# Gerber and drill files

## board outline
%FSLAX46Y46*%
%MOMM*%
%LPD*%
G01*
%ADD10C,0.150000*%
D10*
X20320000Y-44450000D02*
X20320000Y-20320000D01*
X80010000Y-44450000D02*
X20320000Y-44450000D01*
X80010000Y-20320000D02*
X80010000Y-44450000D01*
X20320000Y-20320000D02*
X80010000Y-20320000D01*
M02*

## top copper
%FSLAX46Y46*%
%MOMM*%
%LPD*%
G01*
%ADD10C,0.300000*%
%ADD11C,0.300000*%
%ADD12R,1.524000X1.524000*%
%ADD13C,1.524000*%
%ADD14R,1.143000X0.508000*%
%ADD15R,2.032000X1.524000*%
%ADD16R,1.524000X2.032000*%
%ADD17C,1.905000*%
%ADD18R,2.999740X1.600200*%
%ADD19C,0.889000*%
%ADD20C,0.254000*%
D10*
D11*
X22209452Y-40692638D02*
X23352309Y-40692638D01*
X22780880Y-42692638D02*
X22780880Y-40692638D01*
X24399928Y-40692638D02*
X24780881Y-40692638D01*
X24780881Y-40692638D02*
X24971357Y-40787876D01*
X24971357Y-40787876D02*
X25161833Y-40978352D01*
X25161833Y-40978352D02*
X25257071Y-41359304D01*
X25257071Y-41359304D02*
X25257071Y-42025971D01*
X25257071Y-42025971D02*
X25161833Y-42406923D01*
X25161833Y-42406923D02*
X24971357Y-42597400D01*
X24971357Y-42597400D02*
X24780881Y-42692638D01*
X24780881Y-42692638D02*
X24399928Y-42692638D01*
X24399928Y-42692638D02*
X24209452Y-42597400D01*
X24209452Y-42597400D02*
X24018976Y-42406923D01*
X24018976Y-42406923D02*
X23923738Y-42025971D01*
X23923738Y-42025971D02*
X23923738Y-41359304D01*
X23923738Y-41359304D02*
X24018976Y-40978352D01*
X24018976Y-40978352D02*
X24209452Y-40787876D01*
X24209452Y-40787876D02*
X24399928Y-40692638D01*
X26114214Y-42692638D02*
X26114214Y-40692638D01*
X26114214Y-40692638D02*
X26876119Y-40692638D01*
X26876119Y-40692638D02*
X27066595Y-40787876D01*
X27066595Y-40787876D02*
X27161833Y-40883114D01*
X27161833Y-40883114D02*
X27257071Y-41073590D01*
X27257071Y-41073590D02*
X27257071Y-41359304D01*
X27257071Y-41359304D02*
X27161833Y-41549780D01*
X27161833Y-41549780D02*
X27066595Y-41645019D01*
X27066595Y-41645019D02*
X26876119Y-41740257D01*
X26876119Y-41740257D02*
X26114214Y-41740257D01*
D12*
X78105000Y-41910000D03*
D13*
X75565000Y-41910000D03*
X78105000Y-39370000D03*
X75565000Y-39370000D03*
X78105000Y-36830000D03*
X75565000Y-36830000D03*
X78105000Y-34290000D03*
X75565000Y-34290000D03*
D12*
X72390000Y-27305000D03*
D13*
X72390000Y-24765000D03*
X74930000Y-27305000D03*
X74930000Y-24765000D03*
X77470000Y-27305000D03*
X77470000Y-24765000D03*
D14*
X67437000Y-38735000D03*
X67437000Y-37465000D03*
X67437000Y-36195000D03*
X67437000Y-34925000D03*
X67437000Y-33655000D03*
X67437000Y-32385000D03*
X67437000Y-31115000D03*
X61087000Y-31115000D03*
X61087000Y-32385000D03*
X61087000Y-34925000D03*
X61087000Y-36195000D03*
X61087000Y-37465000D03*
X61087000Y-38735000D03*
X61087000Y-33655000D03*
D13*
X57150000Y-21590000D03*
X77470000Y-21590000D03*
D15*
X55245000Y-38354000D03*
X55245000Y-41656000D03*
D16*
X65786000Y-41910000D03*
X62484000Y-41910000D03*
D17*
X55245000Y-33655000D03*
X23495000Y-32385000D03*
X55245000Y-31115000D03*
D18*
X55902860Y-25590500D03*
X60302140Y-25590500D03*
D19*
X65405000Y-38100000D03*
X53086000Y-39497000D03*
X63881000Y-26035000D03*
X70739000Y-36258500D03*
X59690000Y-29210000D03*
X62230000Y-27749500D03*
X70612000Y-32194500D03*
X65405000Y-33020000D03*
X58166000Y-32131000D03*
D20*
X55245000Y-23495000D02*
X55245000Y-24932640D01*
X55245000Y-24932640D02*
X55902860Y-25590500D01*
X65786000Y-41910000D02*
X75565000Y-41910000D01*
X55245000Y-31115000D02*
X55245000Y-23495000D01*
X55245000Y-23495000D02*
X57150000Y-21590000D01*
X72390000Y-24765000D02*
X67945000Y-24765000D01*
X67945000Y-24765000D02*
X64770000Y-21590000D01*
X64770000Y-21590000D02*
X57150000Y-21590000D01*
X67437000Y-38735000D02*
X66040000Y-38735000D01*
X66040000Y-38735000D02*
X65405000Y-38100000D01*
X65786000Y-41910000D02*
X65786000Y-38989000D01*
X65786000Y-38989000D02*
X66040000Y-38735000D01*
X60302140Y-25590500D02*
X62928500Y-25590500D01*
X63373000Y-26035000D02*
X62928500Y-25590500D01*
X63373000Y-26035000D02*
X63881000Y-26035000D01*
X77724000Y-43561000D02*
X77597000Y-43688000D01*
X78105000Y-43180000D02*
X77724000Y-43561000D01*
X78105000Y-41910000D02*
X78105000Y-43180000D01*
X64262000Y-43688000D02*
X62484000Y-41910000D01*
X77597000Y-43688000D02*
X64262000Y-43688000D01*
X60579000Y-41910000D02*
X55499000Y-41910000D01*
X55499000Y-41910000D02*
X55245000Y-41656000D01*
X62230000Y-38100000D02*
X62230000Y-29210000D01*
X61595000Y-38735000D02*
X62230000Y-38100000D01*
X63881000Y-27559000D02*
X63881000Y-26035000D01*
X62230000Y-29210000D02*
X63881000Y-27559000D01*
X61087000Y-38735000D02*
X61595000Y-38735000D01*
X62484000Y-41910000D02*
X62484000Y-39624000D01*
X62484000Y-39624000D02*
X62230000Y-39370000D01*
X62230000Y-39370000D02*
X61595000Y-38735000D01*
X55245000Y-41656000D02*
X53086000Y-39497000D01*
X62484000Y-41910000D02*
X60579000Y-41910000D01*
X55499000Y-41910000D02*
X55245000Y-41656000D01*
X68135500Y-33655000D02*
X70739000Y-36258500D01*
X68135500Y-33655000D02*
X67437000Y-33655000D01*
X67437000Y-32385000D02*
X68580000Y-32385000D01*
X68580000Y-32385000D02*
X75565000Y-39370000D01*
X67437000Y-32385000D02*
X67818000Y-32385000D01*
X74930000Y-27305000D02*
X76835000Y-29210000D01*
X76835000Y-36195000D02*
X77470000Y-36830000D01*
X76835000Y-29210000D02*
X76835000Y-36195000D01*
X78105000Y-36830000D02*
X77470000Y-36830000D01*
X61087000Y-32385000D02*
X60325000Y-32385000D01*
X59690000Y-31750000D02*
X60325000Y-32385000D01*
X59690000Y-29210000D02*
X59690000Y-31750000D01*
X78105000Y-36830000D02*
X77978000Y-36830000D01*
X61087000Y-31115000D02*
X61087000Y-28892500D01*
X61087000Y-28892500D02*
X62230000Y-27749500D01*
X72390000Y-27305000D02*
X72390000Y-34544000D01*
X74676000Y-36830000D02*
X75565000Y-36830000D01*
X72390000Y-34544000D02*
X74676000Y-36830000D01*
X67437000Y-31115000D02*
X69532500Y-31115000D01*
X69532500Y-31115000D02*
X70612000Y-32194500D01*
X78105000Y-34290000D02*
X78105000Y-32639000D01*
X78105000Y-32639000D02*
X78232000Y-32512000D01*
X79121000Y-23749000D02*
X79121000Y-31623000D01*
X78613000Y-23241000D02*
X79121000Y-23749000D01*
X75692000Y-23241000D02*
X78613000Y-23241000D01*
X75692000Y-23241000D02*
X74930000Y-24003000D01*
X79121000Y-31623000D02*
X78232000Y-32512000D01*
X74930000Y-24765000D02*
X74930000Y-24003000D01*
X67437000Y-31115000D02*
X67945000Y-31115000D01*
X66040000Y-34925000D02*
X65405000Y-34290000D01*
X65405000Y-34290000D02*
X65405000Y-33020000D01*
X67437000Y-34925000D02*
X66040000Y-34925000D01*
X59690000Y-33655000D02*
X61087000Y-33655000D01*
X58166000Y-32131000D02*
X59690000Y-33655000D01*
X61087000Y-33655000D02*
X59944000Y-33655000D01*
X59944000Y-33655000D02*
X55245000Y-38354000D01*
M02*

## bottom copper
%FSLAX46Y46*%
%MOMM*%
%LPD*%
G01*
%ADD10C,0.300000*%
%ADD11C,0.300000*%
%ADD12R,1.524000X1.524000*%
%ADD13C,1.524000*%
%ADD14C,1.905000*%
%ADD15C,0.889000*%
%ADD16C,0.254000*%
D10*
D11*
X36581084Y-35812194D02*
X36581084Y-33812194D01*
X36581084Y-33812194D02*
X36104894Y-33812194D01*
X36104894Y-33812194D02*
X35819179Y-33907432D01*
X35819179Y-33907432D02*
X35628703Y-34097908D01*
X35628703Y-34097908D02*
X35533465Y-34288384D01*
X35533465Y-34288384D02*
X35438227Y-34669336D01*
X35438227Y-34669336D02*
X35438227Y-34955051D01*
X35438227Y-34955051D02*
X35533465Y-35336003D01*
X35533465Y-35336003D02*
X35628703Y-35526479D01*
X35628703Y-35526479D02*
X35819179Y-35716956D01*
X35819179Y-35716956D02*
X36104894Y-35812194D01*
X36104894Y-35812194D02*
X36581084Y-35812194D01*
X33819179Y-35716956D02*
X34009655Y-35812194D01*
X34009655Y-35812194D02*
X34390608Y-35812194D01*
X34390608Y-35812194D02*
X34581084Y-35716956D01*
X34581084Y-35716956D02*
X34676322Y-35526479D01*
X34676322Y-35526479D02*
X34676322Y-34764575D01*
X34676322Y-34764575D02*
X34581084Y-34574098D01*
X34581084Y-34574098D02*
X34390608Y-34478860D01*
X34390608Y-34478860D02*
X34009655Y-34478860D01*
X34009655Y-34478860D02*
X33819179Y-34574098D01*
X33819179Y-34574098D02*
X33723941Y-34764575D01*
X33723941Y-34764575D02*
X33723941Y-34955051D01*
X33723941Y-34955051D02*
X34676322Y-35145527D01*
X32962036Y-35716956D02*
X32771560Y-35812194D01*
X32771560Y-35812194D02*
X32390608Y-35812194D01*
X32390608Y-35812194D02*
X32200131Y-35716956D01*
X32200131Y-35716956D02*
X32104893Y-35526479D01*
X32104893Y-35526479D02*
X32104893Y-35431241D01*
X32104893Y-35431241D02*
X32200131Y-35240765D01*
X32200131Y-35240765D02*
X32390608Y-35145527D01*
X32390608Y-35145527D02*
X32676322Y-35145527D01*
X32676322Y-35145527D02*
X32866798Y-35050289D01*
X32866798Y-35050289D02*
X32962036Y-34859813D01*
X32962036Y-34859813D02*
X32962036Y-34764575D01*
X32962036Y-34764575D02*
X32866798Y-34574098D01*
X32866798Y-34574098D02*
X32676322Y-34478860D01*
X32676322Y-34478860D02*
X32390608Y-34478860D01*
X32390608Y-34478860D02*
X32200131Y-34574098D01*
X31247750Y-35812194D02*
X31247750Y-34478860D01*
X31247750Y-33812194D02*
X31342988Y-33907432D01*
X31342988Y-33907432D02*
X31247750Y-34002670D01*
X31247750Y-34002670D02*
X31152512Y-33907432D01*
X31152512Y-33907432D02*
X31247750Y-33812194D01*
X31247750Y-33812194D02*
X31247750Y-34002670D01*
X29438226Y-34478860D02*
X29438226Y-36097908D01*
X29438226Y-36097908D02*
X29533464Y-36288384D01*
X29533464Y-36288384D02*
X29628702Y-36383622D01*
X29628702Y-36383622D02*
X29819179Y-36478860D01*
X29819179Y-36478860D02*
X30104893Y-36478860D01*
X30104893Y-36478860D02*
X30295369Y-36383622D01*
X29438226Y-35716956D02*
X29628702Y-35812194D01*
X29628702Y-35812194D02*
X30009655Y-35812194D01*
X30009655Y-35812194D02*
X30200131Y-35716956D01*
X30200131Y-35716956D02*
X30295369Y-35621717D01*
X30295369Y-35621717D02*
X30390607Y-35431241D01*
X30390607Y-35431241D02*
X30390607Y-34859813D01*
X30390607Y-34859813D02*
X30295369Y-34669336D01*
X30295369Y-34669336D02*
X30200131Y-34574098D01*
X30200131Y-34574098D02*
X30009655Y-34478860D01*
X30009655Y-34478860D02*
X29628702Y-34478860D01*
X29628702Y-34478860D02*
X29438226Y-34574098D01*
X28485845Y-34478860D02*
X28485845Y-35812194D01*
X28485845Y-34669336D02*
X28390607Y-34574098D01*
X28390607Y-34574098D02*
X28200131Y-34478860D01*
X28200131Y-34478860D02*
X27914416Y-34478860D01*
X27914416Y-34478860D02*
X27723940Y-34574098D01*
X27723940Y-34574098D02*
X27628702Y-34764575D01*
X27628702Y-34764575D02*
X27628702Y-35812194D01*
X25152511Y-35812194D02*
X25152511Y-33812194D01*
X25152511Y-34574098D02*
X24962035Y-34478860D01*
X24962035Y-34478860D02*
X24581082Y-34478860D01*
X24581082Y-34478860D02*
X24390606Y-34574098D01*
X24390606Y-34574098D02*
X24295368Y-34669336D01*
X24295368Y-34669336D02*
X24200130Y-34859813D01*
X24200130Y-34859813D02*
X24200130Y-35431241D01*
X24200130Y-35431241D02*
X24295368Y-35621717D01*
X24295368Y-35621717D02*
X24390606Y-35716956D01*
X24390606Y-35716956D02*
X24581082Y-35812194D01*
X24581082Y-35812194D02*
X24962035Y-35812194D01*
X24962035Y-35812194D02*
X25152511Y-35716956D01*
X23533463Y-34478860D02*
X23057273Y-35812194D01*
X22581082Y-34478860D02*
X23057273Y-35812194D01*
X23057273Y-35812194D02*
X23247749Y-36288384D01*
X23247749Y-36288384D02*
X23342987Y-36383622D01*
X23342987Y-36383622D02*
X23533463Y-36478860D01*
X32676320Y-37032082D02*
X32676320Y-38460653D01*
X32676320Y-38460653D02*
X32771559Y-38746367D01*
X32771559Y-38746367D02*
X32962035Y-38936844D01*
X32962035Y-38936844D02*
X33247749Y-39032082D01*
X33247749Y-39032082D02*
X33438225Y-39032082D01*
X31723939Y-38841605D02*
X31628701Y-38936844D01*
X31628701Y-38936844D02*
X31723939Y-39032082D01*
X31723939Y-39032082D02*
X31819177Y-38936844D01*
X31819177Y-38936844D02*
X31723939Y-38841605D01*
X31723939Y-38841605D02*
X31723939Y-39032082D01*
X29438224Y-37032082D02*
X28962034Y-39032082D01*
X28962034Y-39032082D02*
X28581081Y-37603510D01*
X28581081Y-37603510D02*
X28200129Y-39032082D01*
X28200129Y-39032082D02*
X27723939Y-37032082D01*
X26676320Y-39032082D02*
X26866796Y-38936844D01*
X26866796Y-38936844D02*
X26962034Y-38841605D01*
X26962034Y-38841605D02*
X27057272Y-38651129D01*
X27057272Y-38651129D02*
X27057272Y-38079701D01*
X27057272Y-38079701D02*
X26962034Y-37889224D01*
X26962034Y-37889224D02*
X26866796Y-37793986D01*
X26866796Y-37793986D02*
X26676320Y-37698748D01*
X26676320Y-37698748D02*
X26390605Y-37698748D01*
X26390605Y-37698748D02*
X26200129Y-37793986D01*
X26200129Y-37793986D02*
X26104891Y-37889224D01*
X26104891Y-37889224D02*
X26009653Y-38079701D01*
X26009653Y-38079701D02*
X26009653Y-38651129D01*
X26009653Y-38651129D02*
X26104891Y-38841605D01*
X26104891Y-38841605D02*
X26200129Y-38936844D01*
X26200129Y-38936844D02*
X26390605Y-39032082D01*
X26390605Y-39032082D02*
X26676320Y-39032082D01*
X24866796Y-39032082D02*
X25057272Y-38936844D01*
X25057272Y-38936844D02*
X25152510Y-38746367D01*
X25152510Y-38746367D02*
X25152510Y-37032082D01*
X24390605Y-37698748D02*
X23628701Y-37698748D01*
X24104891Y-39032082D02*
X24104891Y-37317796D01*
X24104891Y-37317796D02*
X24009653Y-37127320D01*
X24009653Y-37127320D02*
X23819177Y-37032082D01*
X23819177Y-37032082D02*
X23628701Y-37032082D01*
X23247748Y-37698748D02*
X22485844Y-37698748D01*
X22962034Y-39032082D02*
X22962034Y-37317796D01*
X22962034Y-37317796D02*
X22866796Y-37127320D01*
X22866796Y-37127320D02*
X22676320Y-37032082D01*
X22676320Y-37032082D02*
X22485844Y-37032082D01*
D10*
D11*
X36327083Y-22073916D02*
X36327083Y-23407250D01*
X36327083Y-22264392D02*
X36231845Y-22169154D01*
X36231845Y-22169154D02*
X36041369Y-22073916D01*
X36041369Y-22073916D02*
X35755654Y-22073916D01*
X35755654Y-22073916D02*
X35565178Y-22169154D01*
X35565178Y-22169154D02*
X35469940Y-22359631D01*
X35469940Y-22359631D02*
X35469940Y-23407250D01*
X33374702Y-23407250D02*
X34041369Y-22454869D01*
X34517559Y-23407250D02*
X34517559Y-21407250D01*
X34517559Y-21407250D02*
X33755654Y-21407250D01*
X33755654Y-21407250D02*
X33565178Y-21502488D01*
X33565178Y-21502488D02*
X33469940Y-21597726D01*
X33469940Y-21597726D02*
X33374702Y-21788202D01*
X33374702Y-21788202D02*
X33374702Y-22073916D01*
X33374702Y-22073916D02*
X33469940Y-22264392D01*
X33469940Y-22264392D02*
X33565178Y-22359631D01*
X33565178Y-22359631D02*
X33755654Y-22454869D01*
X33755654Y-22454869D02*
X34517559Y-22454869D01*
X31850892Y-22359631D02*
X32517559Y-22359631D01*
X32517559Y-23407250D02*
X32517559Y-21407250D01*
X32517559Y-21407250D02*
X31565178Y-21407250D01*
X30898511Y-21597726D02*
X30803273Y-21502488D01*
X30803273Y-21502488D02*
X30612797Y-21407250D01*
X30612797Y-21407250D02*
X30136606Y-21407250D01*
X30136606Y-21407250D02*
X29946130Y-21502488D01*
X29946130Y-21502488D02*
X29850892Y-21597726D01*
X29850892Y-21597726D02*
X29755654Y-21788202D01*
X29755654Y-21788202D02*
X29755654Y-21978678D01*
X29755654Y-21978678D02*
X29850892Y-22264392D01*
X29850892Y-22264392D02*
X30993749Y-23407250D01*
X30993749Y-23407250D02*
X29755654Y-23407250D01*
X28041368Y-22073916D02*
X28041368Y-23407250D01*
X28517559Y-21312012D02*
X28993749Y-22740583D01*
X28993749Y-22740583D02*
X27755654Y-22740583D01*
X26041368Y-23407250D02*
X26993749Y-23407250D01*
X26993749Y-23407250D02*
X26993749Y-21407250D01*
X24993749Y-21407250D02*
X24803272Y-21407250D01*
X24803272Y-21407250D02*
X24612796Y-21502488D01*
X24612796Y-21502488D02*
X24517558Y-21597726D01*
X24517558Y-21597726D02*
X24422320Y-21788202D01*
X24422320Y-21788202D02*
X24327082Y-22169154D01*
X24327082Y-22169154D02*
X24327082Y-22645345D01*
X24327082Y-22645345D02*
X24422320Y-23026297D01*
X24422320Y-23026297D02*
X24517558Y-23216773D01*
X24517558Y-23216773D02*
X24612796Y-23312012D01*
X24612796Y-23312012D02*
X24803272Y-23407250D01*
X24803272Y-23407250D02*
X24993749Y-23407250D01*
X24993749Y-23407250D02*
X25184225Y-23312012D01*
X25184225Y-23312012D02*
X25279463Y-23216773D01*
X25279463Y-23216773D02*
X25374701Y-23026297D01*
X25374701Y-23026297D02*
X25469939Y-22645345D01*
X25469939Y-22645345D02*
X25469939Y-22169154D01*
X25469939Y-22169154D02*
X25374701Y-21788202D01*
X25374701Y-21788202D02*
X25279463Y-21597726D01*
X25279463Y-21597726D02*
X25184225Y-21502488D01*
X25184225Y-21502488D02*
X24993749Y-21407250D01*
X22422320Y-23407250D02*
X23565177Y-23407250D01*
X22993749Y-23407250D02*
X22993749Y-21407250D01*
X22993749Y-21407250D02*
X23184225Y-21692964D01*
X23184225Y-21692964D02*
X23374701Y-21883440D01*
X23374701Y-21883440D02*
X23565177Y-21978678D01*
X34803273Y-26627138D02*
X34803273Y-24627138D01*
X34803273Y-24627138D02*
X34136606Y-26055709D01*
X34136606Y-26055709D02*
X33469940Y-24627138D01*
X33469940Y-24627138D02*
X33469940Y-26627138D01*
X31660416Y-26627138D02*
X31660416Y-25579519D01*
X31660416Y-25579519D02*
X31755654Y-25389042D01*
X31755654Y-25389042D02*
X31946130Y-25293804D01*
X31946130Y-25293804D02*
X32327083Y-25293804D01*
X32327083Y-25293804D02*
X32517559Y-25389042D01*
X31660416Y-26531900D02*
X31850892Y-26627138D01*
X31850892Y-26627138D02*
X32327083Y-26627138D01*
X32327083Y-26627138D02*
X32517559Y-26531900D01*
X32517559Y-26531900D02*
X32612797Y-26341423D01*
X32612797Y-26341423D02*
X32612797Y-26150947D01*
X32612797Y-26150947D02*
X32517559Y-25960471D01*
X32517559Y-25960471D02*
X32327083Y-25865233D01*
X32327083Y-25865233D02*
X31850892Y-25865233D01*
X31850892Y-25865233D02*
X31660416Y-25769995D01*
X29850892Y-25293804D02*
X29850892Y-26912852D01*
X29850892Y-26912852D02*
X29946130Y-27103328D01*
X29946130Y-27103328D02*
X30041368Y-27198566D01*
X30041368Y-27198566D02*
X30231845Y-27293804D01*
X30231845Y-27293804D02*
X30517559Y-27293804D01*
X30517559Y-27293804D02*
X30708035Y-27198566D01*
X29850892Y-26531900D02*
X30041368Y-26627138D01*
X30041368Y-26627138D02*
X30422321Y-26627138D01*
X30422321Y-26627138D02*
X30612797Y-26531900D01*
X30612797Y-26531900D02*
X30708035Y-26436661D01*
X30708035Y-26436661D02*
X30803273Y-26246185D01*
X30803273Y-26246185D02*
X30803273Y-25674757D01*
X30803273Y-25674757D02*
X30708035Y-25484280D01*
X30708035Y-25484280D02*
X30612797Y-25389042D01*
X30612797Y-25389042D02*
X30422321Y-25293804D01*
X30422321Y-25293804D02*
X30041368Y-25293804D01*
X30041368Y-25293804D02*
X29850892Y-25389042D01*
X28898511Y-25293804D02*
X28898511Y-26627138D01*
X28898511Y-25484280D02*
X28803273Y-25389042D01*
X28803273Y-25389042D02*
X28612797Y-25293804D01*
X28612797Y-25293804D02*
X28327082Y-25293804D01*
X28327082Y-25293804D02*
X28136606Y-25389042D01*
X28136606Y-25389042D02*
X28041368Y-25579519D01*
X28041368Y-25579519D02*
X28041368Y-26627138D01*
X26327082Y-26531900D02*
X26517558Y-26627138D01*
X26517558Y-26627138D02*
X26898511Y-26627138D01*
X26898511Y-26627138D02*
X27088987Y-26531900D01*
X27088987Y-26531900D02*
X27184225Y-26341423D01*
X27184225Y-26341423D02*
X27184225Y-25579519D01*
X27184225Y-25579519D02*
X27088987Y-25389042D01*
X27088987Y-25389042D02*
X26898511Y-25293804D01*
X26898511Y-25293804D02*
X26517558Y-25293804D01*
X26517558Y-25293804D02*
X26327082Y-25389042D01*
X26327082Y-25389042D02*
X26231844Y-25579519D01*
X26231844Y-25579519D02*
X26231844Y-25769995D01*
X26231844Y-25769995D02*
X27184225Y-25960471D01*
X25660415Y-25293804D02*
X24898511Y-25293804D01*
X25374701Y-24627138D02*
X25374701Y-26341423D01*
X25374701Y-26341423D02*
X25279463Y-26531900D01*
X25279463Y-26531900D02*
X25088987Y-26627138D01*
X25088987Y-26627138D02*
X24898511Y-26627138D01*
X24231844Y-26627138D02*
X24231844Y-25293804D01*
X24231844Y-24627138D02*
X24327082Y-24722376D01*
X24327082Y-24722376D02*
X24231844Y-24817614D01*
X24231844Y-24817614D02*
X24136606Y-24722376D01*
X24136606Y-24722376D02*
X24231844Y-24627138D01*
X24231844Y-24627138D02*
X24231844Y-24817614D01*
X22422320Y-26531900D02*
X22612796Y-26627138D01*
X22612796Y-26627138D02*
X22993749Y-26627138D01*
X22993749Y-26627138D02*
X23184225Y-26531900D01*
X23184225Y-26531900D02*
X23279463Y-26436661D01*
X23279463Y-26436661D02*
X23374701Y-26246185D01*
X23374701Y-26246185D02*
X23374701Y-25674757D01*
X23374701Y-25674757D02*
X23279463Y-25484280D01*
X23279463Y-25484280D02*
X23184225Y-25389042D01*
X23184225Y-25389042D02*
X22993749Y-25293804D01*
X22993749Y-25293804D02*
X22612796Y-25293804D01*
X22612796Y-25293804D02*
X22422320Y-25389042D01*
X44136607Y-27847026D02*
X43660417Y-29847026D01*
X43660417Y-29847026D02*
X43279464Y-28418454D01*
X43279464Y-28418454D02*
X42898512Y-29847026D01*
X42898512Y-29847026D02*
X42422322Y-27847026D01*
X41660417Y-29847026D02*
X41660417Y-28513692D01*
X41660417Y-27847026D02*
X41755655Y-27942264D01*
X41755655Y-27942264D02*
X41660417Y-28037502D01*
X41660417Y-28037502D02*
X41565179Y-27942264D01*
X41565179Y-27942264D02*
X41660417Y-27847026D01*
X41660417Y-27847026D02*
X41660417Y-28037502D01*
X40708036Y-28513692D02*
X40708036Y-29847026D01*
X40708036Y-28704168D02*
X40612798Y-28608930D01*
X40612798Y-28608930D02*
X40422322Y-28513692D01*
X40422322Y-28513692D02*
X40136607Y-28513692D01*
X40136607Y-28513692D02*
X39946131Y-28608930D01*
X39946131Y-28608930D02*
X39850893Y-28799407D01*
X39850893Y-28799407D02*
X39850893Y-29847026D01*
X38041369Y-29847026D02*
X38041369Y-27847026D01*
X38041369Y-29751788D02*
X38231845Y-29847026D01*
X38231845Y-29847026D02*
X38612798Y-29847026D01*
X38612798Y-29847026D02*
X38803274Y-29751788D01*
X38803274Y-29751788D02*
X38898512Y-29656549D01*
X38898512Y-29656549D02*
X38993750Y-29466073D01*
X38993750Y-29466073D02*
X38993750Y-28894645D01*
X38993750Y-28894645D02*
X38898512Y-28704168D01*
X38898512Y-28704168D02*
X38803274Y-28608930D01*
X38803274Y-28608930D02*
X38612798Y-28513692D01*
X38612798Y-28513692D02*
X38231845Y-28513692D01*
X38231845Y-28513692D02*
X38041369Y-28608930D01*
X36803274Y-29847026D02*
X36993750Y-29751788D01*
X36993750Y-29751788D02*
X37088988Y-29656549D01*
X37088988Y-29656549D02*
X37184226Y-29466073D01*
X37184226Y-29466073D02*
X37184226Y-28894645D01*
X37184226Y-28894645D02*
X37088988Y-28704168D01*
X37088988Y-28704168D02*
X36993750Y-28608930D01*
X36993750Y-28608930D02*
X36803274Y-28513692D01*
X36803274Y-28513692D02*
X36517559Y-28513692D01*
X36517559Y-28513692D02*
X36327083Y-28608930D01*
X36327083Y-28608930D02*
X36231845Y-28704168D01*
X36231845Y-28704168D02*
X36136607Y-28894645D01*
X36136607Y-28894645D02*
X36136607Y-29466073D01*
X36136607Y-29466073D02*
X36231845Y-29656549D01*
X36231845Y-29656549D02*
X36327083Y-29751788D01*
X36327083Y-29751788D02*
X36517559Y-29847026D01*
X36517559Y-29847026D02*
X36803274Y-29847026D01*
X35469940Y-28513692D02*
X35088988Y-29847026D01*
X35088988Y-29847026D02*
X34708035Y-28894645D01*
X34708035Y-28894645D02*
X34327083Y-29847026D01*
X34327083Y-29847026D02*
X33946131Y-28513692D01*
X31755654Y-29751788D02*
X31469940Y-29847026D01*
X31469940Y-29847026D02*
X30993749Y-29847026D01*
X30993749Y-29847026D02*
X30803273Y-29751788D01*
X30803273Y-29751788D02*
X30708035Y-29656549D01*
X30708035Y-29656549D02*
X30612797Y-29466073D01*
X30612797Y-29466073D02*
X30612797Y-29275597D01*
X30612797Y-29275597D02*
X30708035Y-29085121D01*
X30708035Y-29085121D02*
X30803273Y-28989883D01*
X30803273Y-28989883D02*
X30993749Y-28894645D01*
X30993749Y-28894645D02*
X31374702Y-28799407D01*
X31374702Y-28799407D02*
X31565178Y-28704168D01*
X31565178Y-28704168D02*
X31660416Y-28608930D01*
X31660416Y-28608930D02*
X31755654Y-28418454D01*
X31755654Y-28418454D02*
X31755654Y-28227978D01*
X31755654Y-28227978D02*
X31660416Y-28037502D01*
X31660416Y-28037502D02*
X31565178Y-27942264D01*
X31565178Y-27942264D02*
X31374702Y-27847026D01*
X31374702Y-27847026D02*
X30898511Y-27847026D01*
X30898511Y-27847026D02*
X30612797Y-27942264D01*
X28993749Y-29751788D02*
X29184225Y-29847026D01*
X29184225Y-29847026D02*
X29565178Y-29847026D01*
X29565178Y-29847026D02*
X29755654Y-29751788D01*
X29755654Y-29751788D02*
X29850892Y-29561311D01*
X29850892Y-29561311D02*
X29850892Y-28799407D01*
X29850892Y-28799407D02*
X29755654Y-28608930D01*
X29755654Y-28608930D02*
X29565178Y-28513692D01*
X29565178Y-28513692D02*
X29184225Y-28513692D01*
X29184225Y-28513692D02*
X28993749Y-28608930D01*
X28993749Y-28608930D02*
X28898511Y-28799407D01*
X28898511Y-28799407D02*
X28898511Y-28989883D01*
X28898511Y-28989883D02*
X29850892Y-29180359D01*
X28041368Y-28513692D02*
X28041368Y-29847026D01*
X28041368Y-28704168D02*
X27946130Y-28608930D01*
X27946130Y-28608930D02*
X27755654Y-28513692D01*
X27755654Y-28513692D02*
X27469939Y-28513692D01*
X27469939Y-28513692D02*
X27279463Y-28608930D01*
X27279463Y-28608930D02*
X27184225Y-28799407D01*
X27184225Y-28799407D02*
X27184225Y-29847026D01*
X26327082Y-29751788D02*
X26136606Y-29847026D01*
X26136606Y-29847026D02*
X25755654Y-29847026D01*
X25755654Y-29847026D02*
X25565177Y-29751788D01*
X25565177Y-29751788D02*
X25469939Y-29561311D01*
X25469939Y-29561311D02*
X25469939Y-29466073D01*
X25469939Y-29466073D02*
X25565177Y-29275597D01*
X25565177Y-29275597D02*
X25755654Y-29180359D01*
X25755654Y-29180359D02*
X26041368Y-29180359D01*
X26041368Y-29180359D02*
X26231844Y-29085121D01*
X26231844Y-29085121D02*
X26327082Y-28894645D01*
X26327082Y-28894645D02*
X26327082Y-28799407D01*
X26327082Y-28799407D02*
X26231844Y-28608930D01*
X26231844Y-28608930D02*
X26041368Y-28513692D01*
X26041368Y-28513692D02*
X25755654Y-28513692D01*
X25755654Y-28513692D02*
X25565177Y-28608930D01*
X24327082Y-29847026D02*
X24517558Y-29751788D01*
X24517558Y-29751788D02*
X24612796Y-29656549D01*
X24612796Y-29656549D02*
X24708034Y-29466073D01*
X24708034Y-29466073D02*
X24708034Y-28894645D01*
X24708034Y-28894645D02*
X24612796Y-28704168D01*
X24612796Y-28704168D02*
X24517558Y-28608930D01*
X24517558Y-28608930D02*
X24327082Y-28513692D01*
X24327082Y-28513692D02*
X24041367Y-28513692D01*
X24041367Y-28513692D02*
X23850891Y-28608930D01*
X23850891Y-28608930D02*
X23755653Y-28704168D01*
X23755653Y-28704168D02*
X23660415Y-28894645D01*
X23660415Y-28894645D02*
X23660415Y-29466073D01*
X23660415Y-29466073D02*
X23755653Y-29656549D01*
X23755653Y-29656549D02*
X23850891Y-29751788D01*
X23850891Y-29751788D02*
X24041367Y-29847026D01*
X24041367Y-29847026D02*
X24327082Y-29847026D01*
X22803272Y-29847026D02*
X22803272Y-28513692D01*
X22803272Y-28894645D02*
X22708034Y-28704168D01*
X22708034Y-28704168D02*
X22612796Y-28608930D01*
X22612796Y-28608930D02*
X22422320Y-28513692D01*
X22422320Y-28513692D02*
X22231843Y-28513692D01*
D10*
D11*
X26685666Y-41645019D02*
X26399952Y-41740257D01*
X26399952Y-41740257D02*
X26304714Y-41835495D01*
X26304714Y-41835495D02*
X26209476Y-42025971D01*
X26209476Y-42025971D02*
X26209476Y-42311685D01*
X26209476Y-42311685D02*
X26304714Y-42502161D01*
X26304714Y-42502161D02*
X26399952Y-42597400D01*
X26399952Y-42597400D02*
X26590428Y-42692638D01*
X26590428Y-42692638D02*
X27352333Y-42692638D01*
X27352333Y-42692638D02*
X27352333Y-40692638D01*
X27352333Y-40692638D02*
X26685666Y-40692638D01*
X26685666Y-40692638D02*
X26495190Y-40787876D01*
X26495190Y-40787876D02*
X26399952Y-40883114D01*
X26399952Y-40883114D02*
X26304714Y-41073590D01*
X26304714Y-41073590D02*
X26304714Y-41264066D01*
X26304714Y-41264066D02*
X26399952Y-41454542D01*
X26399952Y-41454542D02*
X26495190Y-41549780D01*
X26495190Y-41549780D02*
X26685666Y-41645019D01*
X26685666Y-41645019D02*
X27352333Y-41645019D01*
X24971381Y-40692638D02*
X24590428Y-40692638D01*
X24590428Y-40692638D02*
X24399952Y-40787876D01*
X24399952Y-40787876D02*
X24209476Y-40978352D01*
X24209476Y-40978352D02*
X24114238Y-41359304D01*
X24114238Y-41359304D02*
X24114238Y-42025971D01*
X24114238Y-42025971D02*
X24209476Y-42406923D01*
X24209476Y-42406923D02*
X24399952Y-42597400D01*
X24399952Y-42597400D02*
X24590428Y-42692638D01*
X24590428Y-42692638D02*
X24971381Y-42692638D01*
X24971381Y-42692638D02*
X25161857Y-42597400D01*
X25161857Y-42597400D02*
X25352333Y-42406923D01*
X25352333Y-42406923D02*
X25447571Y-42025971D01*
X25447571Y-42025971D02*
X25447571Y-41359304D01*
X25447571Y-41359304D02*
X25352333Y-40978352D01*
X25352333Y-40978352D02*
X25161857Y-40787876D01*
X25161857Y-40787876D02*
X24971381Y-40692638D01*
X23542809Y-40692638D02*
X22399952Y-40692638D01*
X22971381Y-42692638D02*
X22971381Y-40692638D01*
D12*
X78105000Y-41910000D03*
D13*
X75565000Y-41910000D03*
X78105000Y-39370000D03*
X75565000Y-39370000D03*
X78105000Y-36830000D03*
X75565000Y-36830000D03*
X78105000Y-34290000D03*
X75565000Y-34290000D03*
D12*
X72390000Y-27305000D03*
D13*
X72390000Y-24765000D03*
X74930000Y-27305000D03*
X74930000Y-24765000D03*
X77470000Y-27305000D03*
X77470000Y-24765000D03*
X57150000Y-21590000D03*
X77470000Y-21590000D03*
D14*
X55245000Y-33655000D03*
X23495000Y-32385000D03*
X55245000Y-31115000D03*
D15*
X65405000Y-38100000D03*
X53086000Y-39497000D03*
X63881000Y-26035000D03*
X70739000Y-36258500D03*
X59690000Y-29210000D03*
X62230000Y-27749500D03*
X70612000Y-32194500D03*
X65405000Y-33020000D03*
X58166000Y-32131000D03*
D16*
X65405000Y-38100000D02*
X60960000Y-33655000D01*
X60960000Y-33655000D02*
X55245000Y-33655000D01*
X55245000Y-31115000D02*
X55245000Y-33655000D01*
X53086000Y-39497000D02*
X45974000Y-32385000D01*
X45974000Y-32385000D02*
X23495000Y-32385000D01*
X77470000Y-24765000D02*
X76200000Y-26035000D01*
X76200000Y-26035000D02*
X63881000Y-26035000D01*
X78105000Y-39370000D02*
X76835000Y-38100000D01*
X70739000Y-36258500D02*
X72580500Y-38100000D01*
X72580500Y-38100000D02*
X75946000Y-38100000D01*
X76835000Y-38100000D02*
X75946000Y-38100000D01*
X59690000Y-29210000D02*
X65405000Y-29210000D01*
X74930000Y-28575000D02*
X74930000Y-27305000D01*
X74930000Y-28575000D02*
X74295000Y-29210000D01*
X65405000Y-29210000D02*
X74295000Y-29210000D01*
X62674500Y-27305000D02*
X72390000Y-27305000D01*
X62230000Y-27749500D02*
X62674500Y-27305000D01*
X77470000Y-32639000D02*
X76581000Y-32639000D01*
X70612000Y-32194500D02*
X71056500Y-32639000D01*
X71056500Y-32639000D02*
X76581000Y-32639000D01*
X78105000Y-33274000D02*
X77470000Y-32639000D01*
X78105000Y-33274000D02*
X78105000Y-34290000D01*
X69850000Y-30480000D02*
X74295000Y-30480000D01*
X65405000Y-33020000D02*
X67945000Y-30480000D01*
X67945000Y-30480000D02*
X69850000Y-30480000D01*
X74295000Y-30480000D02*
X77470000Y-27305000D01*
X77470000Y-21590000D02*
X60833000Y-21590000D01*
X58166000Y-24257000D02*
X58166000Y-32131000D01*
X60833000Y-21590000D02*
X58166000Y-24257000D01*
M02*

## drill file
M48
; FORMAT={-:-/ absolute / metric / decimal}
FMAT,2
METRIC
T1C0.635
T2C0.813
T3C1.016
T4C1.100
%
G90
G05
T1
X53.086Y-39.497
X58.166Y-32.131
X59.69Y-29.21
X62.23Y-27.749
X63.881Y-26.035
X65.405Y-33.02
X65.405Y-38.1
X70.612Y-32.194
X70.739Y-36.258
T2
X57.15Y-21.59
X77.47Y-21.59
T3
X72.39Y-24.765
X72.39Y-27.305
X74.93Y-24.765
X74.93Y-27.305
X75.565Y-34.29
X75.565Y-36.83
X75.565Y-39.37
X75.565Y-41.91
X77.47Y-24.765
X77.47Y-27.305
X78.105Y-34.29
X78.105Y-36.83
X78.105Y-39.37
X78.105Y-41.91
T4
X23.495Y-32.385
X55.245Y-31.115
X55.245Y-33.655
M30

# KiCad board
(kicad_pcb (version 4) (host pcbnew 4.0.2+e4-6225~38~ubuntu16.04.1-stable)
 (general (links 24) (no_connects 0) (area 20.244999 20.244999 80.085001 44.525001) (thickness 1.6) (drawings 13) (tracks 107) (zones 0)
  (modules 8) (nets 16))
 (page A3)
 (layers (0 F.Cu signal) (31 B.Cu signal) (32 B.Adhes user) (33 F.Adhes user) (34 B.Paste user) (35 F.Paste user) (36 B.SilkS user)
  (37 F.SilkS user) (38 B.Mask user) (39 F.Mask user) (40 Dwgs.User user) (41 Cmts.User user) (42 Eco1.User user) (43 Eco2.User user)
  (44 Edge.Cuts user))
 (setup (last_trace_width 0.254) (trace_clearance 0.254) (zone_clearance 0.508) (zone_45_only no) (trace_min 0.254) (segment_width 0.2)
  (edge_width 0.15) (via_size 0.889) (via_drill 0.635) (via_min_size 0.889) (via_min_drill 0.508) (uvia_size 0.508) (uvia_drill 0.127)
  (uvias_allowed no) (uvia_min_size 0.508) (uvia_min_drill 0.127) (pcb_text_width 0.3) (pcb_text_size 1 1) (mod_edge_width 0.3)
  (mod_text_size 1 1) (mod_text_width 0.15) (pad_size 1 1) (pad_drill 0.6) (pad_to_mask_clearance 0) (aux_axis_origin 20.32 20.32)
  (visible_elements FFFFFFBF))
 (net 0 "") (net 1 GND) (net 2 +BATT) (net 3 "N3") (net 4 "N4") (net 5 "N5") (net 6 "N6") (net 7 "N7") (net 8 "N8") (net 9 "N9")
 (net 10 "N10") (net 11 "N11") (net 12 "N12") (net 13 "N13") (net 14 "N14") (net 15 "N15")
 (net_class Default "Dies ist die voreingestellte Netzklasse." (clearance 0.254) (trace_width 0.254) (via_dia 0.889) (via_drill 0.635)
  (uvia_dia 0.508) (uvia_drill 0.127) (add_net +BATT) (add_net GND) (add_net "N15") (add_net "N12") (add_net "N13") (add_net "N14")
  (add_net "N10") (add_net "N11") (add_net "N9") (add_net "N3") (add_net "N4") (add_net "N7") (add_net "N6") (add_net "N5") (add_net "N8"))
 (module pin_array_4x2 (layer F.Cu) (at 76.835 38.1 90)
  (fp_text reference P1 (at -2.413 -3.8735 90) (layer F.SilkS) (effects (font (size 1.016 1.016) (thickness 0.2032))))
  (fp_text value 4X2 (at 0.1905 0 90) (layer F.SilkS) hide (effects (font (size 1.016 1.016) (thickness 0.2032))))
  (pad 1 thru_hole rect (at -3.81 1.27 90) (size 1.524 1.524) (drill 1.016) (layers *.Cu *.Mask F.SilkS) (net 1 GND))
  (pad 2 thru_hole circle (at -3.81 -1.27 90) (size 1.524 1.524) (drill 1.016) (layers *.Cu *.Mask F.SilkS) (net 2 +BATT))
  (pad 3 thru_hole circle (at -1.27 1.27 90) (size 1.524 1.524) (drill 1.016) (layers *.Cu *.Mask F.SilkS) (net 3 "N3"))
  (pad 4 thru_hole circle (at -1.27 -1.27 90) (size 1.524 1.524) (drill 1.016) (layers *.Cu *.Mask F.SilkS) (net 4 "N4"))
  (pad 5 thru_hole circle (at 1.27 1.27 90) (size 1.524 1.524) (drill 1.016) (layers *.Cu *.Mask F.SilkS) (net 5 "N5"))
  (pad 6 thru_hole circle (at 1.27 -1.27 90) (size 1.524 1.524) (drill 1.016) (layers *.Cu *.Mask F.SilkS) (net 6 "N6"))
  (pad 7 thru_hole circle (at 3.81 1.27 90) (size 1.524 1.524) (drill 1.016) (layers *.Cu *.Mask F.SilkS) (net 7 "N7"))
  (pad 8 thru_hole circle (at 3.81 -1.27 90) (size 1.524 1.524) (drill 1.016) (layers *.Cu *.Mask F.SilkS) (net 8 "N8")))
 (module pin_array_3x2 (layer F.Cu) (at 74.93 26.035)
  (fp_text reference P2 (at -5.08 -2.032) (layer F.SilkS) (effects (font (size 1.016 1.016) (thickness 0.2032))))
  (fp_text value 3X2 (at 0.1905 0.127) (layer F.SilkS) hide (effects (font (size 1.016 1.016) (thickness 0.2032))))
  (pad 1 thru_hole rect (at -2.54 1.27) (size 1.524 1.524) (drill 1.016) (layers *.Cu *.Mask F.SilkS) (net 6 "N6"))
  (pad 2 thru_hole circle (at -2.54 -1.27) (size 1.524 1.524) (drill 1.016) (layers *.Cu *.Mask F.SilkS) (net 2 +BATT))
  (pad 3 thru_hole circle (at 0 1.27) (size 1.524 1.524) (drill 1.016) (layers *.Cu *.Mask F.SilkS) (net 5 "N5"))
  (pad 4 thru_hole circle (at 0 -1.27) (size 1.524 1.524) (drill 1.016) (layers *.Cu *.Mask F.SilkS) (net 7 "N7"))
  (pad 5 thru_hole circle (at 2.54 1.27) (size 1.524 1.524) (drill 1.016) (layers *.Cu *.Mask F.SilkS) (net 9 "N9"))
  (pad 6 thru_hole circle (at 2.54 -1.27) (size 1.524 1.524) (drill 1.016) (layers *.Cu *.Mask F.SilkS) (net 1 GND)))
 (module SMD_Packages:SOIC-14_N (layer F.Cu) (at 64.135 34.925 90)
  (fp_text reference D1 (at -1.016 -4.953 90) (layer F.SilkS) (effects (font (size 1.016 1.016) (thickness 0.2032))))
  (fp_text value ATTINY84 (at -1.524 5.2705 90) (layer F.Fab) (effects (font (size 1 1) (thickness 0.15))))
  (pad 1 smd rect (at -3.81 3.302 90) (size 0.508 1.143) (layers F.Cu F.Paste F.Mask) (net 2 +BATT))
  (pad 2 smd rect (at -2.54 3.302 90) (size 0.508 1.143) (layers F.Cu F.Paste F.Mask) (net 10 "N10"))
  (pad 3 smd rect (at -1.27 3.302 90) (size 0.508 1.143) (layers F.Cu F.Paste F.Mask) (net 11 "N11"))
  (pad 4 smd rect (at 0 3.302 90) (size 0.508 1.143) (layers F.Cu F.Paste F.Mask) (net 9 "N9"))
  (pad 5 smd rect (at 1.27 3.302 90) (size 0.508 1.143) (layers F.Cu F.Paste F.Mask) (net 3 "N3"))
  (pad 6 smd rect (at 2.54 3.302 90) (size 0.508 1.143) (layers F.Cu F.Paste F.Mask) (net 4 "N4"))
  (pad 7 smd rect (at 3.81 3.302 90) (size 0.508 1.143) (layers F.Cu F.Paste F.Mask) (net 7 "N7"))
  (pad 8 smd rect (at 3.81 -3.048 90) (size 0.508 1.143) (layers F.Cu F.Paste F.Mask) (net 6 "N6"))
  (pad 9 smd rect (at 2.54 -3.048 90) (size 0.508 1.143) (layers F.Cu F.Paste F.Mask) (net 5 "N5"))
  (pad 11 smd rect (at 0 -3.048 90) (size 0.508 1.143) (layers F.Cu F.Paste F.Mask) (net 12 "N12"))
  (pad 12 smd rect (at -1.27 -3.048 90) (size 0.508 1.143) (layers F.Cu F.Paste F.Mask) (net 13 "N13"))
  (pad 13 smd rect (at -2.54 -3.048 90) (size 0.508 1.143) (layers F.Cu F.Paste F.Mask) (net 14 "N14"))
  (pad 14 smd rect (at -3.81 -3.048 90) (size 0.508 1.143) (layers F.Cu F.Paste F.Mask) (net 1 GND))
  (pad 10 smd rect (at 1.27 -3.048 90) (size 0.508 1.143) (layers F.Cu F.Paste F.Mask) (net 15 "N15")))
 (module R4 (layer F.Cu) (at 67.31 21.59) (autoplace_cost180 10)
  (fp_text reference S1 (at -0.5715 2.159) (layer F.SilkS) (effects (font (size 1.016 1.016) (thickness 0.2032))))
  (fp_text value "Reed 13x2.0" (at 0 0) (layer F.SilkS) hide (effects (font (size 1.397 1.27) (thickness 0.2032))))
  (pad 1 thru_hole circle (at -10.16 0) (size 1.524 1.524) (drill 0.8128) (layers *.Cu *.Mask F.SilkS) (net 2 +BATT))
  (pad 2 thru_hole circle (at 10.16 0) (size 1.524 1.524) (drill 0.8128) (layers *.Cu *.Mask F.SilkS) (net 15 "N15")))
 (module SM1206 (layer F.Cu) (at 55.245 40.005 270)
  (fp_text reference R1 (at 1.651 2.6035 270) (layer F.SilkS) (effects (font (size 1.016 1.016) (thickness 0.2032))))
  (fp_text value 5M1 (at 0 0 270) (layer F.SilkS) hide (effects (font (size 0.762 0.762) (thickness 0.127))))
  (pad 1 smd rect (at -1.651 0 270) (size 1.524 2.032) (layers F.Cu F.Paste F.Mask) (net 15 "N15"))
  (pad 2 smd rect (at 1.651 0 270) (size 1.524 2.032) (layers F.Cu F.Paste F.Mask) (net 1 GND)))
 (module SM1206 (layer F.Cu) (at 64.135 41.91 180)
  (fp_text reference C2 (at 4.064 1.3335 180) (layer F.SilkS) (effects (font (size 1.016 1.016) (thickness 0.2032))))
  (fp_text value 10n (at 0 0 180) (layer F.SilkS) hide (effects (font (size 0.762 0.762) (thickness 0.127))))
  (pad 1 smd rect (at -1.651 0 180) (size 1.524 2.032) (layers F.Cu F.Paste F.Mask) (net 2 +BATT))
  (pad 2 smd rect (at 1.651 0 180) (size 1.524 2.032) (layers F.Cu F.Paste F.Mask) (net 1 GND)))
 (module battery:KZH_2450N (layer F.Cu) (at 39.37 32.385 180)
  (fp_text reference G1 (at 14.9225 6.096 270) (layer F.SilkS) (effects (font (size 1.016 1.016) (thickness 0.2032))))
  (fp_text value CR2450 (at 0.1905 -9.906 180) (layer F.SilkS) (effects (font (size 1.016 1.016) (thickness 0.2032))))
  (pad 1 thru_hole circle (at -15.875 -1.27 180) (size 1.905 1.905) (drill 1.1) (layers *.Cu *.Mask F.SilkS) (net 2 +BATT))
  (pad 2 thru_hole circle (at 15.875 0 180) (size 1.905 1.905) (drill 1.1) (layers *.Cu *.Mask F.SilkS) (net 1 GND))
  (pad 1 thru_hole circle (at -15.875 1.27 180) (size 1.905 1.905) (drill 1.1) (layers *.Cu *.Mask F.SilkS) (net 2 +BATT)))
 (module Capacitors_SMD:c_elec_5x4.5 (layer F.Cu) (at 58.1025 25.5905 180)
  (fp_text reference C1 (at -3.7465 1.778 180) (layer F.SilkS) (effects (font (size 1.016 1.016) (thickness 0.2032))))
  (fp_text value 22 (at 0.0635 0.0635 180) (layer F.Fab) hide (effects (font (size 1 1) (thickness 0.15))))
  (pad 1 smd rect (at 2.19964 0 180) (size 2.99974 1.6002) (layers F.Cu F.Paste F.Mask) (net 2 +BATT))
  (pad 2 smd rect (at -2.19964 0 180) (size 2.99974 1.6002) (layers F.Cu F.Paste F.Mask) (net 1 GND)))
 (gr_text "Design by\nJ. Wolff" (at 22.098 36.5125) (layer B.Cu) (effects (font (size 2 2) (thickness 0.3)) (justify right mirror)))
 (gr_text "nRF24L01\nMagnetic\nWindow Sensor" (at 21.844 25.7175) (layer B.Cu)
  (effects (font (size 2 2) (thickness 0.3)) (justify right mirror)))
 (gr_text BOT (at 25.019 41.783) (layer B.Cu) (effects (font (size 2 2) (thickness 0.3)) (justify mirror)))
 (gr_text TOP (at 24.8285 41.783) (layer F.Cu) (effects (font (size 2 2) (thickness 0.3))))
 (gr_line (start 20.32 44.45) (end 20.32 20.32) (angle 90) (layer Edge.Cuts) (width 0.15))
 (gr_line (start 80.01 44.45) (end 20.32 44.45) (angle 90) (layer Edge.Cuts) (width 0.15))
 (gr_line (start 80.01 20.32) (end 80.01 44.45) (angle 90) (layer Edge.Cuts) (width 0.15))
 (gr_line (start 20.32 20.32) (end 80.01 20.32) (angle 90) (layer Edge.Cuts) (width 0.15))
 (segment (start 55.245 23.495) (end 55.245 24.93264) (width 0.254) (layer F.Cu) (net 2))
 (segment (start 55.245 24.93264) (end 55.90286 25.5905) (width 0.254) (layer F.Cu) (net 2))
 (segment (start 65.786 41.91) (end 75.565 41.91) (width 0.254) (layer F.Cu) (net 2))
 (segment (start 55.245 31.115) (end 55.245 23.495) (width 0.254) (layer F.Cu) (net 2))
 (segment (start 55.245 23.495) (end 57.15 21.59) (width 0.254) (layer F.Cu) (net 2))
 (segment (start 72.39 24.765) (end 67.945 24.765) (width 0.254) (layer F.Cu) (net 2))
 (segment (start 67.945 24.765) (end 64.77 21.59) (width 0.254) (layer F.Cu) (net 2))
 (segment (start 64.77 21.59) (end 57.15 21.59) (width 0.254) (layer F.Cu) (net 2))
 (segment (start 67.437 38.735) (end 66.04 38.735) (width 0.254) (layer F.Cu) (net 2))
 (segment (start 66.04 38.735) (end 65.405 38.1) (width 0.254) (layer F.Cu) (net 2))
 (via (at 65.405 38.1) (size 0.889) (drill 0.635) (layers F.Cu B.Cu) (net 2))
 (segment (start 65.405 38.1) (end 60.96 33.655) (width 0.254) (layer B.Cu) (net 2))
 (segment (start 60.96 33.655) (end 55.245 33.655) (width 0.254) (layer B.Cu) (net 2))
 (segment (start 65.786 41.91) (end 65.786 38.989) (width 0.254) (layer F.Cu) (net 2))
 (segment (start 65.786 38.989) (end 66.04 38.735) (width 0.254) (layer F.Cu) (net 2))
 (segment (start 55.245 31.115) (end 55.245 33.655) (width 0.254) (layer B.Cu) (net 2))
 (segment (start 60.30214 25.5905) (end 62.9285 25.5905) (width 0.254) (layer F.Cu) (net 1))
 (segment (start 63.373 26.035) (end 62.9285 25.5905) (width 0.254) (layer F.Cu) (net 1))
 (segment (start 63.373 26.035) (end 63.881 26.035) (width 0.254) (layer F.Cu) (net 1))
 (segment (start 77.724 43.561) (end 77.597 43.688) (width 0.254) (layer F.Cu) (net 1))
 (segment (start 78.105 43.18) (end 77.724 43.561) (width 0.254) (layer F.Cu) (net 1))
 (segment (start 78.105 41.91) (end 78.105 43.18) (width 0.254) (layer F.Cu) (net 1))
 (segment (start 64.262 43.688) (end 62.484 41.91) (width 0.254) (layer F.Cu) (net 1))
 (segment (start 77.597 43.688) (end 64.262 43.688) (width 0.254) (layer F.Cu) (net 1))
 (segment (start 60.579 41.91) (end 55.499 41.91) (width 0.254) (layer F.Cu) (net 1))
 (segment (start 55.499 41.91) (end 55.245 41.656) (width 0.254) (layer F.Cu) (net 1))
 (segment (start 62.23 38.1) (end 62.23 29.21) (width 0.254) (layer F.Cu) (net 1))
 (segment (start 61.595 38.735) (end 62.23 38.1) (width 0.254) (layer F.Cu) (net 1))
 (segment (start 63.881 27.559) (end 63.881 26.035) (width 0.254) (layer F.Cu) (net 1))
 (segment (start 62.23 29.21) (end 63.881 27.559) (width 0.254) (layer F.Cu) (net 1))
 (segment (start 61.087 38.735) (end 61.595 38.735) (width 0.254) (layer F.Cu) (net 1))
 (segment (start 62.484 41.91) (end 62.484 39.624) (width 0.254) (layer F.Cu) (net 1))
 (segment (start 62.484 39.624) (end 62.23 39.37) (width 0.254) (layer F.Cu) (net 1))
 (segment (start 62.23 39.37) (end 61.595 38.735) (width 0.254) (layer F.Cu) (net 1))
 (segment (start 55.245 41.656) (end 53.086 39.497) (width 0.254) (layer F.Cu) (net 1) (status 80000))
 (via (at 53.086 39.497) (size 0.889) (layers F.Cu B.Cu) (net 1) (status 80000))
 (segment (start 53.086 39.497) (end 45.974 32.385) (width 0.254) (layer B.Cu) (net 1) (status 80000))
 (segment (start 45.974 32.385) (end 23.495 32.385) (width 0.254) (layer B.Cu) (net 1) (status 80000))
 (segment (start 77.47 24.765) (end 76.2 26.035) (width 0.254) (layer B.Cu) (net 1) (status 80000))
 (via (at 63.881 26.035) (size 0.889) (layers F.Cu B.Cu) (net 1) (status 80000))
 (segment (start 76.2 26.035) (end 63.881 26.035) (width 0.254) (layer B.Cu) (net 1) (status 80000))
 (segment (start 62.484 41.91) (end 60.579 41.91) (width 0.254) (layer F.Cu) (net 1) (status 80000))
 (segment (start 55.499 41.91) (end 55.245 41.656) (width 0.254) (layer F.Cu) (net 1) (status 80000))
 (segment (start 78.105 39.37) (end 76.835 38.1) (width 0.254) (layer B.Cu) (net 3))
 (segment (start 68.1355 33.655) (end 70.739 36.2585) (width 0.254) (layer F.Cu) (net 3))
 (via (at 70.739 36.2585) (size 0.889) (drill 0.635) (layers F.Cu B.Cu) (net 3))
 (segment (start 70.739 36.2585) (end 72.5805 38.1) (width 0.254) (layer B.Cu) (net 3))
 (segment (start 72.5805 38.1) (end 75.946 38.1) (width 0.254) (layer B.Cu) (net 3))
 (segment (start 68.1355 33.655) (end 67.437 33.655) (width 0.254) (layer F.Cu) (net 3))
 (segment (start 76.835 38.1) (end 75.946 38.1) (width 0.254) (layer B.Cu) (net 3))
 (segment (start 67.437 32.385) (end 68.58 32.385) (width 0.254) (layer F.Cu) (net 4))
 (segment (start 68.58 32.385) (end 75.565 39.37) (width 0.254) (layer F.Cu) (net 4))
 (segment (start 67.437 32.385) (end 67.818 32.385) (width 0.254) (layer F.Cu) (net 4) (status 80000))
 (segment (start 74.93 27.305) (end 76.835 29.21) (width 0.254) (layer F.Cu) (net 5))
 (segment (start 76.835 36.195) (end 77.47 36.83) (width 0.254) (layer F.Cu) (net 5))
 (segment (start 76.835 29.21) (end 76.835 36.195) (width 0.254) (layer F.Cu) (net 5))
 (segment (start 78.105 36.83) (end 77.47 36.83) (width 0.254) (layer F.Cu) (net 5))
 (segment (start 61.087 32.385) (end 60.325 32.385) (width 0.254) (layer F.Cu) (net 5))
 (segment (start 59.69 31.75) (end 60.325 32.385) (width 0.254) (layer F.Cu) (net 5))
 (segment (start 59.69 29.21) (end 65.405 29.21) (width 0.254) (layer B.Cu) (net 5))
 (segment (start 74.93 28.575) (end 74.93 27.305) (width 0.254) (layer B.Cu) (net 5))
 (segment (start 74.93 28.575) (end 74.295 29.21) (width 0.254) (layer B.Cu) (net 5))
 (segment (start 65.405 29.21) (end 74.295 29.21) (width 0.254) (layer B.Cu) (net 5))
 (via (at 59.69 29.21) (size 0.889) (drill 0.635) (layers F.Cu B.Cu) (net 5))
 (segment (start 59.69 29.21) (end 59.69 31.75) (width 0.254) (layer F.Cu) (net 5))
 (segment (start 78.105 36.83) (end 77.978 36.83) (width 0.254) (layer F.Cu) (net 5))
 (segment (start 61.087 31.115) (end 61.087 28.8925) (width 0.254) (layer F.Cu) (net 6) (status 400000))
 (segment (start 62.6745 27.305) (end 72.39 27.305) (width 0.254) (layer B.Cu) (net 6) (status 800000))
 (segment (start 62.23 27.7495) (end 62.6745 27.305) (width 0.254) (layer B.Cu) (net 6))
 (via (at 62.23 27.7495) (size 0.889) (drill 0.635) (layers F.Cu B.Cu) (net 6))
 (segment (start 61.087 28.8925) (end 62.23 27.7495) (width 0.254) (layer F.Cu) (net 6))
 (segment (start 72.39 27.305) (end 72.39 34.544) (width 0.254) (layer F.Cu) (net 6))
 (segment (start 74.676 36.83) (end 75.565 36.83) (width 0.254) (layer F.Cu) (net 6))
 (segment (start 72.39 34.544) (end 74.676 36.83) (width 0.254) (layer F.Cu) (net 6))
 (segment (start 77.47 32.639) (end 76.581 32.639) (width 0.254) (layer B.Cu) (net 7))
 (segment (start 70.612 32.1945) (end 71.0565 32.639) (width 0.254) (layer B.Cu) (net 7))
 (segment (start 71.0565 32.639) (end 76.581 32.639) (width 0.254) (layer B.Cu) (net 7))
 (segment (start 67.437 31.115) (end 69.5325 31.115) (width 0.254) (layer F.Cu) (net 7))
 (segment (start 69.5325 31.115) (end 70.612 32.1945) (width 0.254) (layer F.Cu) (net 7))
 (via (at 70.612 32.1945) (size 0.889) (drill 0.635) (layers F.Cu B.Cu) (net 7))
 (segment (start 78.105 33.274) (end 77.47 32.639) (width 0.254) (layer B.Cu) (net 7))
 (segment (start 78.105 33.274) (end 78.105 34.29) (width 0.254) (layer B.Cu) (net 7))
 (segment (start 78.105 34.29) (end 78.105 32.639) (width 0.254) (layer F.Cu) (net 7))
 (segment (start 78.105 32.639) (end 78.232 32.512) (width 0.254) (layer F.Cu) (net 7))
 (segment (start 79.121 23.749) (end 79.121 31.623) (width 0.254) (layer F.Cu) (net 7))
 (segment (start 78.613 23.241) (end 79.121 23.749) (width 0.254) (layer F.Cu) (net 7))
 (segment (start 75.692 23.241) (end 78.613 23.241) (width 0.254) (layer F.Cu) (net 7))
 (segment (start 75.692 23.241) (end 74.93 24.003) (width 0.254) (layer F.Cu) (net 7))
 (segment (start 79.121 31.623) (end 78.232 32.512) (width 0.254) (layer F.Cu) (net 7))
 (segment (start 74.93 24.765) (end 74.93 24.003) (width 0.254) (layer F.Cu) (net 7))
 (segment (start 67.437 31.115) (end 67.945 31.115) (width 0.254) (layer F.Cu) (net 7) (status 80000))
 (segment (start 69.85 30.48) (end 74.295 30.48) (width 0.254) (layer B.Cu) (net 9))
 (segment (start 66.04 34.925) (end 65.405 34.29) (width 0.254) (layer F.Cu) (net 9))
 (segment (start 65.405 34.29) (end 65.405 33.02) (width 0.254) (layer F.Cu) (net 9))
 (via (at 65.405 33.02) (size 0.889) (drill 0.635) (layers F.Cu B.Cu) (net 9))
 (segment (start 65.405 33.02) (end 67.945 30.48) (width 0.254) (layer B.Cu) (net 9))
 (segment (start 67.945 30.48) (end 69.85 30.48) (width 0.254) (layer B.Cu) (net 9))
 (segment (start 67.437 34.925) (end 66.04 34.925) (width 0.254) (layer F.Cu) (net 9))
 (segment (start 74.295 30.48) (end 77.47 27.305) (width 0.254) (layer B.Cu) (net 9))
 (segment (start 77.47 21.59) (end 60.833 21.59) (width 0.254) (layer B.Cu) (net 15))
 (segment (start 59.69 33.655) (end 61.087 33.655) (width 0.254) (layer F.Cu) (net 15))
 (segment (start 58.166 32.131) (end 59.69 33.655) (width 0.254) (layer F.Cu) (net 15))
 (via (at 58.166 32.131) (size 0.889) (drill 0.635) (layers F.Cu B.Cu) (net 15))
 (segment (start 58.166 24.257) (end 58.166 32.131) (width 0.254) (layer B.Cu) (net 15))
 (segment (start 60.833 21.59) (end 58.166 24.257) (width 0.254) (layer B.Cu) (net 15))
 (segment (start 61.087 33.655) (end 59.944 33.655) (width 0.254) (layer F.Cu) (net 15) (status 80000))
 (segment (start 59.944 33.655) (end 55.245 38.354) (width 0.254) (layer F.Cu) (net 15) (status 80000)))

